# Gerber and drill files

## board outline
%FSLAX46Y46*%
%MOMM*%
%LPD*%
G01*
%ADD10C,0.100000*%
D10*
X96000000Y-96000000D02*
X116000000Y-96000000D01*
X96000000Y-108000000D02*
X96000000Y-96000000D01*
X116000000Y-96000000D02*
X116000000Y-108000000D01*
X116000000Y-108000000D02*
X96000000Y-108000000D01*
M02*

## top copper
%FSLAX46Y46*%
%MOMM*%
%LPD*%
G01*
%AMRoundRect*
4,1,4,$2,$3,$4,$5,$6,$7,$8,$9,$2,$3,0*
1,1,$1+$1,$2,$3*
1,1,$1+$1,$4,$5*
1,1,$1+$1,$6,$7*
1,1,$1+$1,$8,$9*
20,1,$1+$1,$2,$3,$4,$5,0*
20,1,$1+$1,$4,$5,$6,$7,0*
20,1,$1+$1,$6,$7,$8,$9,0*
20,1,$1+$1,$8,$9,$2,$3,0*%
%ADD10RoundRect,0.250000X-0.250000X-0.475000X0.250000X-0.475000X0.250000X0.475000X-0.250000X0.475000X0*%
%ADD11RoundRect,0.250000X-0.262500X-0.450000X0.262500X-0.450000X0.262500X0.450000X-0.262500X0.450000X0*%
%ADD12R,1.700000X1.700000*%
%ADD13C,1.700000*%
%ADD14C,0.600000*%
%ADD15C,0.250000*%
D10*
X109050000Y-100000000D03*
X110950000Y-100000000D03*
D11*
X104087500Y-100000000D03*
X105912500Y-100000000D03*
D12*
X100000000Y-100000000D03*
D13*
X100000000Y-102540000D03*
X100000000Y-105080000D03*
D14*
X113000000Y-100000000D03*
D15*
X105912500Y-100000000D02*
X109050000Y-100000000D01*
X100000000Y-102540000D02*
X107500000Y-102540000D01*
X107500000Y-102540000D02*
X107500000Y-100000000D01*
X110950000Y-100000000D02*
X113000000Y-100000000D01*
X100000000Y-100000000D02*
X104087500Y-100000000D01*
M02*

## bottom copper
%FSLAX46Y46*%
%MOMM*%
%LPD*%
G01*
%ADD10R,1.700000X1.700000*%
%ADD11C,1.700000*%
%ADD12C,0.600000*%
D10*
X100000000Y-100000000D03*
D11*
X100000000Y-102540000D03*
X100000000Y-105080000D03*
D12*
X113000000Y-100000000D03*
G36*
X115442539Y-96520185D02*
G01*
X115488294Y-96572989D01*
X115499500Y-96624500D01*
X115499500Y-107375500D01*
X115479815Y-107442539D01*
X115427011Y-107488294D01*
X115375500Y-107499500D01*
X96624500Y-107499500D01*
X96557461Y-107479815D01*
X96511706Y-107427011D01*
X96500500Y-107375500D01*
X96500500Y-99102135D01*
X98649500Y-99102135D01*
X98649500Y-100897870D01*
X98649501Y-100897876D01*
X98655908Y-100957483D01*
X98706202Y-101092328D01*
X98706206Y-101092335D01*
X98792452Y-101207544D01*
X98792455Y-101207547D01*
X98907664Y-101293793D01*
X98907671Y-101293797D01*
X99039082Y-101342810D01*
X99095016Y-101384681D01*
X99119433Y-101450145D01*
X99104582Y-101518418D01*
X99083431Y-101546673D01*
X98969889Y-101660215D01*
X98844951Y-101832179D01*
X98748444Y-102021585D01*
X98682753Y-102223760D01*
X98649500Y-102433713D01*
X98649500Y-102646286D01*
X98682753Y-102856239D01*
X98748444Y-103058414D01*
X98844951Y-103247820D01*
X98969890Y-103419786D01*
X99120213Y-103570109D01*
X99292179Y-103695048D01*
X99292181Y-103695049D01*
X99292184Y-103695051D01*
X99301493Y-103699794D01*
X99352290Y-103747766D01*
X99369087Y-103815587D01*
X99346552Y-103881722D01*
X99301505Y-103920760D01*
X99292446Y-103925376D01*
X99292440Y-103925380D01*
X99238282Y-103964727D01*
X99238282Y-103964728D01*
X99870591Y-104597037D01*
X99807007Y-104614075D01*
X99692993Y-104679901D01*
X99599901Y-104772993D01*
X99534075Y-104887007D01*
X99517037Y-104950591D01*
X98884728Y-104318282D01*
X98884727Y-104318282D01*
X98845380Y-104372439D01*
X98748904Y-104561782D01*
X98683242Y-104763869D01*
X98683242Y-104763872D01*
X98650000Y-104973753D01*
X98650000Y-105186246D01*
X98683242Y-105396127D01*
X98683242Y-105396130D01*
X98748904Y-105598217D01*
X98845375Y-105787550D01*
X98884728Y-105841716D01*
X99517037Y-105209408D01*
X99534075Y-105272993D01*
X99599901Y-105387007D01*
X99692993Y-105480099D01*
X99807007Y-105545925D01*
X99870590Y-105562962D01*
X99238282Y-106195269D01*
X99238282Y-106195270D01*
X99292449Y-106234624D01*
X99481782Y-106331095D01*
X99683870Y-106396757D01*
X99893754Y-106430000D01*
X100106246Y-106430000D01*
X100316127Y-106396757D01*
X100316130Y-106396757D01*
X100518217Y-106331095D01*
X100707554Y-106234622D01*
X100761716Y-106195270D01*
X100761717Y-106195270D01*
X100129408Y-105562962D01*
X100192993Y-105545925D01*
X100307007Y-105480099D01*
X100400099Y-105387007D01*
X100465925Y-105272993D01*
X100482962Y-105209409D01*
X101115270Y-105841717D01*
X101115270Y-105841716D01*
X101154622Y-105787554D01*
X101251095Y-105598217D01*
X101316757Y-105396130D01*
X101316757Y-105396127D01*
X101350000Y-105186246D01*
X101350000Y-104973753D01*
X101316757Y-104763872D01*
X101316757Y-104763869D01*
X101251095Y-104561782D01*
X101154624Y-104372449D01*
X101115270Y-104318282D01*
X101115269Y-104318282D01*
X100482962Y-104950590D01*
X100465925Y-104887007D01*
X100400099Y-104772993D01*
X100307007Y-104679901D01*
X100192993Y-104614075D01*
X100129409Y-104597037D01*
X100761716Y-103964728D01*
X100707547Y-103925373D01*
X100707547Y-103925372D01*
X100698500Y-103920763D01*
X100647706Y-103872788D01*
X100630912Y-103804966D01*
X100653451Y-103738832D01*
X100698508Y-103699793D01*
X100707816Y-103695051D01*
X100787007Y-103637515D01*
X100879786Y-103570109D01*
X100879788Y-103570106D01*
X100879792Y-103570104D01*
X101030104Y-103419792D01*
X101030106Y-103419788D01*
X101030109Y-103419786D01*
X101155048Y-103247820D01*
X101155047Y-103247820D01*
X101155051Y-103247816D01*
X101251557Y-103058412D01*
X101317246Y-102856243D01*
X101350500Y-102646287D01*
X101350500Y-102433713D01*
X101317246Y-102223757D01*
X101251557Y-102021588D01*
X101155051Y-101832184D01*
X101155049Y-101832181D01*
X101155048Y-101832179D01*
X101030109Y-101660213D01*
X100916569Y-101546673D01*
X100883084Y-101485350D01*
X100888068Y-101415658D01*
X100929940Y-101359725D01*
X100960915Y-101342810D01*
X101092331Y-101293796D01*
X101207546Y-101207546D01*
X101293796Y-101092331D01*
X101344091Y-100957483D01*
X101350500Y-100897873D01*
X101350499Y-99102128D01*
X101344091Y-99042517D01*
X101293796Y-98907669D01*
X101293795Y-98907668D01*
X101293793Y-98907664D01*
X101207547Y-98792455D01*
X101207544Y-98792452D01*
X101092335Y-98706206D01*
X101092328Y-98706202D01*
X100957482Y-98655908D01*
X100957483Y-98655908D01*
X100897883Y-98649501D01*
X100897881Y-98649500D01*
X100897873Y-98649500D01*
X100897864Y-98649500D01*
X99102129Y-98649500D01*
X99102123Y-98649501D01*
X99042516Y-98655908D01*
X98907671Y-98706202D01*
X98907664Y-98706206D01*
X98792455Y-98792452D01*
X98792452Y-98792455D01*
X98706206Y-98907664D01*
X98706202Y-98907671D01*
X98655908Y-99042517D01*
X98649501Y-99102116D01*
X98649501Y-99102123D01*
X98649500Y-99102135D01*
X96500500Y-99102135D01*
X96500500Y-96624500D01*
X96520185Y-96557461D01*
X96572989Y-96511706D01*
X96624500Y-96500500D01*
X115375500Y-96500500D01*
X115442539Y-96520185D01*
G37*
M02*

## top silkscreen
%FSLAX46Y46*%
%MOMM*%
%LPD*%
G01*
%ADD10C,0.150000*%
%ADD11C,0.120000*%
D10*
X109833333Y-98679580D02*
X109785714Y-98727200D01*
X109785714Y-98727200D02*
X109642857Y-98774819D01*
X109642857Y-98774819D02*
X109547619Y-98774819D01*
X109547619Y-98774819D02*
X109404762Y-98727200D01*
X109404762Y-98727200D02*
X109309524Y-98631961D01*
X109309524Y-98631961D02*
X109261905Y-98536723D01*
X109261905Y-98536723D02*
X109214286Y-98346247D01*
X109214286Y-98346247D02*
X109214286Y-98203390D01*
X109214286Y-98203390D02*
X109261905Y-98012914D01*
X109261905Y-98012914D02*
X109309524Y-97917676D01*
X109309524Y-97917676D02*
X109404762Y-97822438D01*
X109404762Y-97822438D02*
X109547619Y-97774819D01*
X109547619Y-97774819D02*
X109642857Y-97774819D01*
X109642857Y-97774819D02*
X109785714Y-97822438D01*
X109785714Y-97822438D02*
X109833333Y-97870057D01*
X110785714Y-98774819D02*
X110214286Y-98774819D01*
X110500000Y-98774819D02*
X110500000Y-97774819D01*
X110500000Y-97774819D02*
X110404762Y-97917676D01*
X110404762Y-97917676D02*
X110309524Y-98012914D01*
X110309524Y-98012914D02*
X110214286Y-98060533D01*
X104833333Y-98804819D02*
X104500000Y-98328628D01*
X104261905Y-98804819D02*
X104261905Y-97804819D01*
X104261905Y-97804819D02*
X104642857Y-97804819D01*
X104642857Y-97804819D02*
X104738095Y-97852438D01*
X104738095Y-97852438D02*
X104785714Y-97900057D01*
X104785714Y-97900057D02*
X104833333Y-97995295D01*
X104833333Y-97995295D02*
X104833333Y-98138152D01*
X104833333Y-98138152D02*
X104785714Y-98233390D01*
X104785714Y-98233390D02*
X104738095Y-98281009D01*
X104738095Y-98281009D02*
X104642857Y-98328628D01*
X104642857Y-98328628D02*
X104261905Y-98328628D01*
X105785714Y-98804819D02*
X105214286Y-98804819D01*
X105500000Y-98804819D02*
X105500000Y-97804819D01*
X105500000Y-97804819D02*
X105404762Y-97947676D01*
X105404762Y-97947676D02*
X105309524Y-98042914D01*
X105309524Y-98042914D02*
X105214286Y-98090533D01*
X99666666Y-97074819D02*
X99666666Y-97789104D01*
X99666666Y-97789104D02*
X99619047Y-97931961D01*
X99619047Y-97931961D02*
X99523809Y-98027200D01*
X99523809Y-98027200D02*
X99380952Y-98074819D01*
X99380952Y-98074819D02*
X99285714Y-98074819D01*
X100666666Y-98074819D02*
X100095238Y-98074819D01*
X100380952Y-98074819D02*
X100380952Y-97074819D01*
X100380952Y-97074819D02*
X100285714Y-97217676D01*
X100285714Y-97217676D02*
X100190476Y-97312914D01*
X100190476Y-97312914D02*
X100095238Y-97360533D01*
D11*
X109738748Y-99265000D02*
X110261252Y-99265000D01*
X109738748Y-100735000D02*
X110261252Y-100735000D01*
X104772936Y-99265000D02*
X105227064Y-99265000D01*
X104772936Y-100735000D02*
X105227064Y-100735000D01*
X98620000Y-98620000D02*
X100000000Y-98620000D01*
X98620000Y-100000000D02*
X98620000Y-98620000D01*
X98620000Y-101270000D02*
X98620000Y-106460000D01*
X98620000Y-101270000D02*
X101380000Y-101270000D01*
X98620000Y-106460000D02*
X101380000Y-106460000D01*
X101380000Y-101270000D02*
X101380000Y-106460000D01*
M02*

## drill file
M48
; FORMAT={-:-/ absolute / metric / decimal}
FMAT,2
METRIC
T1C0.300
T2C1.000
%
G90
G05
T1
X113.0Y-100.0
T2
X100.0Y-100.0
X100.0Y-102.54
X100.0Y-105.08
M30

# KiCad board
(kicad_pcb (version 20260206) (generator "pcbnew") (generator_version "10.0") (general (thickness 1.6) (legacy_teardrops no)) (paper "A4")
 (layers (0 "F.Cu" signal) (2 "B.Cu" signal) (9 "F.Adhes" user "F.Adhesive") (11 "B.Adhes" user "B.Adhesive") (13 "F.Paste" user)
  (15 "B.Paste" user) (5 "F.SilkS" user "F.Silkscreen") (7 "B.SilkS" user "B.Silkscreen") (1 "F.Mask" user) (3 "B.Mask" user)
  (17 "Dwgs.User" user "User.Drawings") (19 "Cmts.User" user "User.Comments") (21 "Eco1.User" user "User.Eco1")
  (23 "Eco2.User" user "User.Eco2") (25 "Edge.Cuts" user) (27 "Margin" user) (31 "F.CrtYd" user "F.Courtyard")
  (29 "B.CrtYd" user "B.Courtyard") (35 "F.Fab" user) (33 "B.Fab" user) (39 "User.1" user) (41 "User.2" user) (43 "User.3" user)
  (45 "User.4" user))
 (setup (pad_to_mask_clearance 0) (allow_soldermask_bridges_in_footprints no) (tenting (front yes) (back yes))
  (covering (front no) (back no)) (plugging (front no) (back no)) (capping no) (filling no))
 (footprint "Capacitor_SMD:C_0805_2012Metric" (layer "F.Cu") (at 110 100)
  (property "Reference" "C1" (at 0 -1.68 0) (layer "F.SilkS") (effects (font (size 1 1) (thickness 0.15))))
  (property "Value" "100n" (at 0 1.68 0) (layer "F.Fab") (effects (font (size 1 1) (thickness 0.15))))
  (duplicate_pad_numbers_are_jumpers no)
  (fp_line (start -0.261252 -0.735) (end 0.261252 -0.735) (stroke (width 0.12) (type solid)) (layer "F.SilkS"))
  (fp_line (start -0.261252 0.735) (end 0.261252 0.735) (stroke (width 0.12) (type solid)) (layer "F.SilkS"))
  (pad "1" smd roundrect (at -0.95 0) (size 1 1.45) (layers "F.Cu" "F.Mask" "F.Paste") (roundrect_rratio 0.25) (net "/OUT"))
  (pad "2" smd roundrect (at 0.95 0) (size 1 1.45) (layers "F.Cu" "F.Mask" "F.Paste") (roundrect_rratio 0.25) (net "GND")))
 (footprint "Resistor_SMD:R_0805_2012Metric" (layer "F.Cu") (at 105 100)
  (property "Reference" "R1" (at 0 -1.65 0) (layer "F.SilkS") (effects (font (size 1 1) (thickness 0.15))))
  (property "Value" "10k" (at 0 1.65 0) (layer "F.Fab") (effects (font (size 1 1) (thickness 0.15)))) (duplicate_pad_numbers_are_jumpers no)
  (fp_line (start -0.227064 -0.735) (end 0.227064 -0.735) (stroke (width 0.12) (type solid)) (layer "F.SilkS"))
  (fp_line (start -0.227064 0.735) (end 0.227064 0.735) (stroke (width 0.12) (type solid)) (layer "F.SilkS"))
  (pad "1" smd roundrect (at -0.9125 0) (size 1.025 1.4) (layers "F.Cu" "F.Mask" "F.Paste") (roundrect_rratio 0.243902) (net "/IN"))
  (pad "2" smd roundrect (at 0.9125 0) (size 1.025 1.4) (layers "F.Cu" "F.Mask" "F.Paste") (roundrect_rratio 0.243902) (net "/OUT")))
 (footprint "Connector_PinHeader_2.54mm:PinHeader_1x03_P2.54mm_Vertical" (layer "F.Cu") (at 100 100)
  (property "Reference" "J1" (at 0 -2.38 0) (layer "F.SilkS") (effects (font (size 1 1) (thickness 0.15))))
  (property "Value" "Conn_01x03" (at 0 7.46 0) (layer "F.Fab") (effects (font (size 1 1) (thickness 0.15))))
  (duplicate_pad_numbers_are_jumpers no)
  (fp_line (start -1.38 -1.38) (end 0 -1.38) (stroke (width 0.12) (type solid)) (layer "F.SilkS"))
  (fp_line (start -1.38 0) (end -1.38 -1.38) (stroke (width 0.12) (type solid)) (layer "F.SilkS"))
  (fp_line (start -1.38 1.27) (end -1.38 6.46) (stroke (width 0.12) (type solid)) (layer "F.SilkS"))
  (fp_line (start -1.38 1.27) (end 1.38 1.27) (stroke (width 0.12) (type solid)) (layer "F.SilkS"))
  (fp_line (start -1.38 6.46) (end 1.38 6.46) (stroke (width 0.12) (type solid)) (layer "F.SilkS"))
  (fp_line (start 1.38 1.27) (end 1.38 6.46) (stroke (width 0.12) (type solid)) (layer "F.SilkS"))
  (pad "1" thru_hole rect (at 0 0) (size 1.7 1.7) (drill 1) (layers "*.Cu" "*.Mask") (remove_unused_layers no) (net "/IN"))
  (pad "2" thru_hole circle (at 0 2.54) (size 1.7 1.7) (drill 1) (layers "*.Cu" "*.Mask") (remove_unused_layers no) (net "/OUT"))
  (pad "3" thru_hole circle (at 0 5.08) (size 1.7 1.7) (drill 1) (layers "*.Cu" "*.Mask") (remove_unused_layers no) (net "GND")))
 (gr_line (start 96 96) (end 116 96) (stroke (width 0.1) (type default)) (layer "Edge.Cuts"))
 (gr_line (start 96 108) (end 96 96) (stroke (width 0.1) (type default)) (layer "Edge.Cuts"))
 (gr_line (start 116 96) (end 116 108) (stroke (width 0.1) (type default)) (layer "Edge.Cuts"))
 (gr_line (start 116 108) (end 96 108) (stroke (width 0.1) (type default)) (layer "Edge.Cuts"))
 (segment (start 105.9125 100) (end 109.05 100) (width 0.25) (layer "F.Cu") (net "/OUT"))
 (segment (start 100 102.54) (end 107.5 102.54) (width 0.25) (layer "F.Cu") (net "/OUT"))
 (segment (start 107.5 102.54) (end 107.5 100) (width 0.25) (layer "F.Cu") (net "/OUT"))
 (segment (start 110.95 100) (end 113 100) (width 0.25) (layer "F.Cu") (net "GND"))
 (via (at 113 100) (size 0.6) (drill 0.3) (layers "F.Cu" "B.Cu") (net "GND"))
 (segment (start 100 100) (end 104.0875 100) (width 0.25) (layer "F.Cu") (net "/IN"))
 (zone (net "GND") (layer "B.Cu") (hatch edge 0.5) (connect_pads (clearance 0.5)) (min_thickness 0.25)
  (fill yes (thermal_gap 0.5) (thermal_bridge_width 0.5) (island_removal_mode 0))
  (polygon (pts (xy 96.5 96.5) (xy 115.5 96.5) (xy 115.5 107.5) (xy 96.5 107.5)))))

